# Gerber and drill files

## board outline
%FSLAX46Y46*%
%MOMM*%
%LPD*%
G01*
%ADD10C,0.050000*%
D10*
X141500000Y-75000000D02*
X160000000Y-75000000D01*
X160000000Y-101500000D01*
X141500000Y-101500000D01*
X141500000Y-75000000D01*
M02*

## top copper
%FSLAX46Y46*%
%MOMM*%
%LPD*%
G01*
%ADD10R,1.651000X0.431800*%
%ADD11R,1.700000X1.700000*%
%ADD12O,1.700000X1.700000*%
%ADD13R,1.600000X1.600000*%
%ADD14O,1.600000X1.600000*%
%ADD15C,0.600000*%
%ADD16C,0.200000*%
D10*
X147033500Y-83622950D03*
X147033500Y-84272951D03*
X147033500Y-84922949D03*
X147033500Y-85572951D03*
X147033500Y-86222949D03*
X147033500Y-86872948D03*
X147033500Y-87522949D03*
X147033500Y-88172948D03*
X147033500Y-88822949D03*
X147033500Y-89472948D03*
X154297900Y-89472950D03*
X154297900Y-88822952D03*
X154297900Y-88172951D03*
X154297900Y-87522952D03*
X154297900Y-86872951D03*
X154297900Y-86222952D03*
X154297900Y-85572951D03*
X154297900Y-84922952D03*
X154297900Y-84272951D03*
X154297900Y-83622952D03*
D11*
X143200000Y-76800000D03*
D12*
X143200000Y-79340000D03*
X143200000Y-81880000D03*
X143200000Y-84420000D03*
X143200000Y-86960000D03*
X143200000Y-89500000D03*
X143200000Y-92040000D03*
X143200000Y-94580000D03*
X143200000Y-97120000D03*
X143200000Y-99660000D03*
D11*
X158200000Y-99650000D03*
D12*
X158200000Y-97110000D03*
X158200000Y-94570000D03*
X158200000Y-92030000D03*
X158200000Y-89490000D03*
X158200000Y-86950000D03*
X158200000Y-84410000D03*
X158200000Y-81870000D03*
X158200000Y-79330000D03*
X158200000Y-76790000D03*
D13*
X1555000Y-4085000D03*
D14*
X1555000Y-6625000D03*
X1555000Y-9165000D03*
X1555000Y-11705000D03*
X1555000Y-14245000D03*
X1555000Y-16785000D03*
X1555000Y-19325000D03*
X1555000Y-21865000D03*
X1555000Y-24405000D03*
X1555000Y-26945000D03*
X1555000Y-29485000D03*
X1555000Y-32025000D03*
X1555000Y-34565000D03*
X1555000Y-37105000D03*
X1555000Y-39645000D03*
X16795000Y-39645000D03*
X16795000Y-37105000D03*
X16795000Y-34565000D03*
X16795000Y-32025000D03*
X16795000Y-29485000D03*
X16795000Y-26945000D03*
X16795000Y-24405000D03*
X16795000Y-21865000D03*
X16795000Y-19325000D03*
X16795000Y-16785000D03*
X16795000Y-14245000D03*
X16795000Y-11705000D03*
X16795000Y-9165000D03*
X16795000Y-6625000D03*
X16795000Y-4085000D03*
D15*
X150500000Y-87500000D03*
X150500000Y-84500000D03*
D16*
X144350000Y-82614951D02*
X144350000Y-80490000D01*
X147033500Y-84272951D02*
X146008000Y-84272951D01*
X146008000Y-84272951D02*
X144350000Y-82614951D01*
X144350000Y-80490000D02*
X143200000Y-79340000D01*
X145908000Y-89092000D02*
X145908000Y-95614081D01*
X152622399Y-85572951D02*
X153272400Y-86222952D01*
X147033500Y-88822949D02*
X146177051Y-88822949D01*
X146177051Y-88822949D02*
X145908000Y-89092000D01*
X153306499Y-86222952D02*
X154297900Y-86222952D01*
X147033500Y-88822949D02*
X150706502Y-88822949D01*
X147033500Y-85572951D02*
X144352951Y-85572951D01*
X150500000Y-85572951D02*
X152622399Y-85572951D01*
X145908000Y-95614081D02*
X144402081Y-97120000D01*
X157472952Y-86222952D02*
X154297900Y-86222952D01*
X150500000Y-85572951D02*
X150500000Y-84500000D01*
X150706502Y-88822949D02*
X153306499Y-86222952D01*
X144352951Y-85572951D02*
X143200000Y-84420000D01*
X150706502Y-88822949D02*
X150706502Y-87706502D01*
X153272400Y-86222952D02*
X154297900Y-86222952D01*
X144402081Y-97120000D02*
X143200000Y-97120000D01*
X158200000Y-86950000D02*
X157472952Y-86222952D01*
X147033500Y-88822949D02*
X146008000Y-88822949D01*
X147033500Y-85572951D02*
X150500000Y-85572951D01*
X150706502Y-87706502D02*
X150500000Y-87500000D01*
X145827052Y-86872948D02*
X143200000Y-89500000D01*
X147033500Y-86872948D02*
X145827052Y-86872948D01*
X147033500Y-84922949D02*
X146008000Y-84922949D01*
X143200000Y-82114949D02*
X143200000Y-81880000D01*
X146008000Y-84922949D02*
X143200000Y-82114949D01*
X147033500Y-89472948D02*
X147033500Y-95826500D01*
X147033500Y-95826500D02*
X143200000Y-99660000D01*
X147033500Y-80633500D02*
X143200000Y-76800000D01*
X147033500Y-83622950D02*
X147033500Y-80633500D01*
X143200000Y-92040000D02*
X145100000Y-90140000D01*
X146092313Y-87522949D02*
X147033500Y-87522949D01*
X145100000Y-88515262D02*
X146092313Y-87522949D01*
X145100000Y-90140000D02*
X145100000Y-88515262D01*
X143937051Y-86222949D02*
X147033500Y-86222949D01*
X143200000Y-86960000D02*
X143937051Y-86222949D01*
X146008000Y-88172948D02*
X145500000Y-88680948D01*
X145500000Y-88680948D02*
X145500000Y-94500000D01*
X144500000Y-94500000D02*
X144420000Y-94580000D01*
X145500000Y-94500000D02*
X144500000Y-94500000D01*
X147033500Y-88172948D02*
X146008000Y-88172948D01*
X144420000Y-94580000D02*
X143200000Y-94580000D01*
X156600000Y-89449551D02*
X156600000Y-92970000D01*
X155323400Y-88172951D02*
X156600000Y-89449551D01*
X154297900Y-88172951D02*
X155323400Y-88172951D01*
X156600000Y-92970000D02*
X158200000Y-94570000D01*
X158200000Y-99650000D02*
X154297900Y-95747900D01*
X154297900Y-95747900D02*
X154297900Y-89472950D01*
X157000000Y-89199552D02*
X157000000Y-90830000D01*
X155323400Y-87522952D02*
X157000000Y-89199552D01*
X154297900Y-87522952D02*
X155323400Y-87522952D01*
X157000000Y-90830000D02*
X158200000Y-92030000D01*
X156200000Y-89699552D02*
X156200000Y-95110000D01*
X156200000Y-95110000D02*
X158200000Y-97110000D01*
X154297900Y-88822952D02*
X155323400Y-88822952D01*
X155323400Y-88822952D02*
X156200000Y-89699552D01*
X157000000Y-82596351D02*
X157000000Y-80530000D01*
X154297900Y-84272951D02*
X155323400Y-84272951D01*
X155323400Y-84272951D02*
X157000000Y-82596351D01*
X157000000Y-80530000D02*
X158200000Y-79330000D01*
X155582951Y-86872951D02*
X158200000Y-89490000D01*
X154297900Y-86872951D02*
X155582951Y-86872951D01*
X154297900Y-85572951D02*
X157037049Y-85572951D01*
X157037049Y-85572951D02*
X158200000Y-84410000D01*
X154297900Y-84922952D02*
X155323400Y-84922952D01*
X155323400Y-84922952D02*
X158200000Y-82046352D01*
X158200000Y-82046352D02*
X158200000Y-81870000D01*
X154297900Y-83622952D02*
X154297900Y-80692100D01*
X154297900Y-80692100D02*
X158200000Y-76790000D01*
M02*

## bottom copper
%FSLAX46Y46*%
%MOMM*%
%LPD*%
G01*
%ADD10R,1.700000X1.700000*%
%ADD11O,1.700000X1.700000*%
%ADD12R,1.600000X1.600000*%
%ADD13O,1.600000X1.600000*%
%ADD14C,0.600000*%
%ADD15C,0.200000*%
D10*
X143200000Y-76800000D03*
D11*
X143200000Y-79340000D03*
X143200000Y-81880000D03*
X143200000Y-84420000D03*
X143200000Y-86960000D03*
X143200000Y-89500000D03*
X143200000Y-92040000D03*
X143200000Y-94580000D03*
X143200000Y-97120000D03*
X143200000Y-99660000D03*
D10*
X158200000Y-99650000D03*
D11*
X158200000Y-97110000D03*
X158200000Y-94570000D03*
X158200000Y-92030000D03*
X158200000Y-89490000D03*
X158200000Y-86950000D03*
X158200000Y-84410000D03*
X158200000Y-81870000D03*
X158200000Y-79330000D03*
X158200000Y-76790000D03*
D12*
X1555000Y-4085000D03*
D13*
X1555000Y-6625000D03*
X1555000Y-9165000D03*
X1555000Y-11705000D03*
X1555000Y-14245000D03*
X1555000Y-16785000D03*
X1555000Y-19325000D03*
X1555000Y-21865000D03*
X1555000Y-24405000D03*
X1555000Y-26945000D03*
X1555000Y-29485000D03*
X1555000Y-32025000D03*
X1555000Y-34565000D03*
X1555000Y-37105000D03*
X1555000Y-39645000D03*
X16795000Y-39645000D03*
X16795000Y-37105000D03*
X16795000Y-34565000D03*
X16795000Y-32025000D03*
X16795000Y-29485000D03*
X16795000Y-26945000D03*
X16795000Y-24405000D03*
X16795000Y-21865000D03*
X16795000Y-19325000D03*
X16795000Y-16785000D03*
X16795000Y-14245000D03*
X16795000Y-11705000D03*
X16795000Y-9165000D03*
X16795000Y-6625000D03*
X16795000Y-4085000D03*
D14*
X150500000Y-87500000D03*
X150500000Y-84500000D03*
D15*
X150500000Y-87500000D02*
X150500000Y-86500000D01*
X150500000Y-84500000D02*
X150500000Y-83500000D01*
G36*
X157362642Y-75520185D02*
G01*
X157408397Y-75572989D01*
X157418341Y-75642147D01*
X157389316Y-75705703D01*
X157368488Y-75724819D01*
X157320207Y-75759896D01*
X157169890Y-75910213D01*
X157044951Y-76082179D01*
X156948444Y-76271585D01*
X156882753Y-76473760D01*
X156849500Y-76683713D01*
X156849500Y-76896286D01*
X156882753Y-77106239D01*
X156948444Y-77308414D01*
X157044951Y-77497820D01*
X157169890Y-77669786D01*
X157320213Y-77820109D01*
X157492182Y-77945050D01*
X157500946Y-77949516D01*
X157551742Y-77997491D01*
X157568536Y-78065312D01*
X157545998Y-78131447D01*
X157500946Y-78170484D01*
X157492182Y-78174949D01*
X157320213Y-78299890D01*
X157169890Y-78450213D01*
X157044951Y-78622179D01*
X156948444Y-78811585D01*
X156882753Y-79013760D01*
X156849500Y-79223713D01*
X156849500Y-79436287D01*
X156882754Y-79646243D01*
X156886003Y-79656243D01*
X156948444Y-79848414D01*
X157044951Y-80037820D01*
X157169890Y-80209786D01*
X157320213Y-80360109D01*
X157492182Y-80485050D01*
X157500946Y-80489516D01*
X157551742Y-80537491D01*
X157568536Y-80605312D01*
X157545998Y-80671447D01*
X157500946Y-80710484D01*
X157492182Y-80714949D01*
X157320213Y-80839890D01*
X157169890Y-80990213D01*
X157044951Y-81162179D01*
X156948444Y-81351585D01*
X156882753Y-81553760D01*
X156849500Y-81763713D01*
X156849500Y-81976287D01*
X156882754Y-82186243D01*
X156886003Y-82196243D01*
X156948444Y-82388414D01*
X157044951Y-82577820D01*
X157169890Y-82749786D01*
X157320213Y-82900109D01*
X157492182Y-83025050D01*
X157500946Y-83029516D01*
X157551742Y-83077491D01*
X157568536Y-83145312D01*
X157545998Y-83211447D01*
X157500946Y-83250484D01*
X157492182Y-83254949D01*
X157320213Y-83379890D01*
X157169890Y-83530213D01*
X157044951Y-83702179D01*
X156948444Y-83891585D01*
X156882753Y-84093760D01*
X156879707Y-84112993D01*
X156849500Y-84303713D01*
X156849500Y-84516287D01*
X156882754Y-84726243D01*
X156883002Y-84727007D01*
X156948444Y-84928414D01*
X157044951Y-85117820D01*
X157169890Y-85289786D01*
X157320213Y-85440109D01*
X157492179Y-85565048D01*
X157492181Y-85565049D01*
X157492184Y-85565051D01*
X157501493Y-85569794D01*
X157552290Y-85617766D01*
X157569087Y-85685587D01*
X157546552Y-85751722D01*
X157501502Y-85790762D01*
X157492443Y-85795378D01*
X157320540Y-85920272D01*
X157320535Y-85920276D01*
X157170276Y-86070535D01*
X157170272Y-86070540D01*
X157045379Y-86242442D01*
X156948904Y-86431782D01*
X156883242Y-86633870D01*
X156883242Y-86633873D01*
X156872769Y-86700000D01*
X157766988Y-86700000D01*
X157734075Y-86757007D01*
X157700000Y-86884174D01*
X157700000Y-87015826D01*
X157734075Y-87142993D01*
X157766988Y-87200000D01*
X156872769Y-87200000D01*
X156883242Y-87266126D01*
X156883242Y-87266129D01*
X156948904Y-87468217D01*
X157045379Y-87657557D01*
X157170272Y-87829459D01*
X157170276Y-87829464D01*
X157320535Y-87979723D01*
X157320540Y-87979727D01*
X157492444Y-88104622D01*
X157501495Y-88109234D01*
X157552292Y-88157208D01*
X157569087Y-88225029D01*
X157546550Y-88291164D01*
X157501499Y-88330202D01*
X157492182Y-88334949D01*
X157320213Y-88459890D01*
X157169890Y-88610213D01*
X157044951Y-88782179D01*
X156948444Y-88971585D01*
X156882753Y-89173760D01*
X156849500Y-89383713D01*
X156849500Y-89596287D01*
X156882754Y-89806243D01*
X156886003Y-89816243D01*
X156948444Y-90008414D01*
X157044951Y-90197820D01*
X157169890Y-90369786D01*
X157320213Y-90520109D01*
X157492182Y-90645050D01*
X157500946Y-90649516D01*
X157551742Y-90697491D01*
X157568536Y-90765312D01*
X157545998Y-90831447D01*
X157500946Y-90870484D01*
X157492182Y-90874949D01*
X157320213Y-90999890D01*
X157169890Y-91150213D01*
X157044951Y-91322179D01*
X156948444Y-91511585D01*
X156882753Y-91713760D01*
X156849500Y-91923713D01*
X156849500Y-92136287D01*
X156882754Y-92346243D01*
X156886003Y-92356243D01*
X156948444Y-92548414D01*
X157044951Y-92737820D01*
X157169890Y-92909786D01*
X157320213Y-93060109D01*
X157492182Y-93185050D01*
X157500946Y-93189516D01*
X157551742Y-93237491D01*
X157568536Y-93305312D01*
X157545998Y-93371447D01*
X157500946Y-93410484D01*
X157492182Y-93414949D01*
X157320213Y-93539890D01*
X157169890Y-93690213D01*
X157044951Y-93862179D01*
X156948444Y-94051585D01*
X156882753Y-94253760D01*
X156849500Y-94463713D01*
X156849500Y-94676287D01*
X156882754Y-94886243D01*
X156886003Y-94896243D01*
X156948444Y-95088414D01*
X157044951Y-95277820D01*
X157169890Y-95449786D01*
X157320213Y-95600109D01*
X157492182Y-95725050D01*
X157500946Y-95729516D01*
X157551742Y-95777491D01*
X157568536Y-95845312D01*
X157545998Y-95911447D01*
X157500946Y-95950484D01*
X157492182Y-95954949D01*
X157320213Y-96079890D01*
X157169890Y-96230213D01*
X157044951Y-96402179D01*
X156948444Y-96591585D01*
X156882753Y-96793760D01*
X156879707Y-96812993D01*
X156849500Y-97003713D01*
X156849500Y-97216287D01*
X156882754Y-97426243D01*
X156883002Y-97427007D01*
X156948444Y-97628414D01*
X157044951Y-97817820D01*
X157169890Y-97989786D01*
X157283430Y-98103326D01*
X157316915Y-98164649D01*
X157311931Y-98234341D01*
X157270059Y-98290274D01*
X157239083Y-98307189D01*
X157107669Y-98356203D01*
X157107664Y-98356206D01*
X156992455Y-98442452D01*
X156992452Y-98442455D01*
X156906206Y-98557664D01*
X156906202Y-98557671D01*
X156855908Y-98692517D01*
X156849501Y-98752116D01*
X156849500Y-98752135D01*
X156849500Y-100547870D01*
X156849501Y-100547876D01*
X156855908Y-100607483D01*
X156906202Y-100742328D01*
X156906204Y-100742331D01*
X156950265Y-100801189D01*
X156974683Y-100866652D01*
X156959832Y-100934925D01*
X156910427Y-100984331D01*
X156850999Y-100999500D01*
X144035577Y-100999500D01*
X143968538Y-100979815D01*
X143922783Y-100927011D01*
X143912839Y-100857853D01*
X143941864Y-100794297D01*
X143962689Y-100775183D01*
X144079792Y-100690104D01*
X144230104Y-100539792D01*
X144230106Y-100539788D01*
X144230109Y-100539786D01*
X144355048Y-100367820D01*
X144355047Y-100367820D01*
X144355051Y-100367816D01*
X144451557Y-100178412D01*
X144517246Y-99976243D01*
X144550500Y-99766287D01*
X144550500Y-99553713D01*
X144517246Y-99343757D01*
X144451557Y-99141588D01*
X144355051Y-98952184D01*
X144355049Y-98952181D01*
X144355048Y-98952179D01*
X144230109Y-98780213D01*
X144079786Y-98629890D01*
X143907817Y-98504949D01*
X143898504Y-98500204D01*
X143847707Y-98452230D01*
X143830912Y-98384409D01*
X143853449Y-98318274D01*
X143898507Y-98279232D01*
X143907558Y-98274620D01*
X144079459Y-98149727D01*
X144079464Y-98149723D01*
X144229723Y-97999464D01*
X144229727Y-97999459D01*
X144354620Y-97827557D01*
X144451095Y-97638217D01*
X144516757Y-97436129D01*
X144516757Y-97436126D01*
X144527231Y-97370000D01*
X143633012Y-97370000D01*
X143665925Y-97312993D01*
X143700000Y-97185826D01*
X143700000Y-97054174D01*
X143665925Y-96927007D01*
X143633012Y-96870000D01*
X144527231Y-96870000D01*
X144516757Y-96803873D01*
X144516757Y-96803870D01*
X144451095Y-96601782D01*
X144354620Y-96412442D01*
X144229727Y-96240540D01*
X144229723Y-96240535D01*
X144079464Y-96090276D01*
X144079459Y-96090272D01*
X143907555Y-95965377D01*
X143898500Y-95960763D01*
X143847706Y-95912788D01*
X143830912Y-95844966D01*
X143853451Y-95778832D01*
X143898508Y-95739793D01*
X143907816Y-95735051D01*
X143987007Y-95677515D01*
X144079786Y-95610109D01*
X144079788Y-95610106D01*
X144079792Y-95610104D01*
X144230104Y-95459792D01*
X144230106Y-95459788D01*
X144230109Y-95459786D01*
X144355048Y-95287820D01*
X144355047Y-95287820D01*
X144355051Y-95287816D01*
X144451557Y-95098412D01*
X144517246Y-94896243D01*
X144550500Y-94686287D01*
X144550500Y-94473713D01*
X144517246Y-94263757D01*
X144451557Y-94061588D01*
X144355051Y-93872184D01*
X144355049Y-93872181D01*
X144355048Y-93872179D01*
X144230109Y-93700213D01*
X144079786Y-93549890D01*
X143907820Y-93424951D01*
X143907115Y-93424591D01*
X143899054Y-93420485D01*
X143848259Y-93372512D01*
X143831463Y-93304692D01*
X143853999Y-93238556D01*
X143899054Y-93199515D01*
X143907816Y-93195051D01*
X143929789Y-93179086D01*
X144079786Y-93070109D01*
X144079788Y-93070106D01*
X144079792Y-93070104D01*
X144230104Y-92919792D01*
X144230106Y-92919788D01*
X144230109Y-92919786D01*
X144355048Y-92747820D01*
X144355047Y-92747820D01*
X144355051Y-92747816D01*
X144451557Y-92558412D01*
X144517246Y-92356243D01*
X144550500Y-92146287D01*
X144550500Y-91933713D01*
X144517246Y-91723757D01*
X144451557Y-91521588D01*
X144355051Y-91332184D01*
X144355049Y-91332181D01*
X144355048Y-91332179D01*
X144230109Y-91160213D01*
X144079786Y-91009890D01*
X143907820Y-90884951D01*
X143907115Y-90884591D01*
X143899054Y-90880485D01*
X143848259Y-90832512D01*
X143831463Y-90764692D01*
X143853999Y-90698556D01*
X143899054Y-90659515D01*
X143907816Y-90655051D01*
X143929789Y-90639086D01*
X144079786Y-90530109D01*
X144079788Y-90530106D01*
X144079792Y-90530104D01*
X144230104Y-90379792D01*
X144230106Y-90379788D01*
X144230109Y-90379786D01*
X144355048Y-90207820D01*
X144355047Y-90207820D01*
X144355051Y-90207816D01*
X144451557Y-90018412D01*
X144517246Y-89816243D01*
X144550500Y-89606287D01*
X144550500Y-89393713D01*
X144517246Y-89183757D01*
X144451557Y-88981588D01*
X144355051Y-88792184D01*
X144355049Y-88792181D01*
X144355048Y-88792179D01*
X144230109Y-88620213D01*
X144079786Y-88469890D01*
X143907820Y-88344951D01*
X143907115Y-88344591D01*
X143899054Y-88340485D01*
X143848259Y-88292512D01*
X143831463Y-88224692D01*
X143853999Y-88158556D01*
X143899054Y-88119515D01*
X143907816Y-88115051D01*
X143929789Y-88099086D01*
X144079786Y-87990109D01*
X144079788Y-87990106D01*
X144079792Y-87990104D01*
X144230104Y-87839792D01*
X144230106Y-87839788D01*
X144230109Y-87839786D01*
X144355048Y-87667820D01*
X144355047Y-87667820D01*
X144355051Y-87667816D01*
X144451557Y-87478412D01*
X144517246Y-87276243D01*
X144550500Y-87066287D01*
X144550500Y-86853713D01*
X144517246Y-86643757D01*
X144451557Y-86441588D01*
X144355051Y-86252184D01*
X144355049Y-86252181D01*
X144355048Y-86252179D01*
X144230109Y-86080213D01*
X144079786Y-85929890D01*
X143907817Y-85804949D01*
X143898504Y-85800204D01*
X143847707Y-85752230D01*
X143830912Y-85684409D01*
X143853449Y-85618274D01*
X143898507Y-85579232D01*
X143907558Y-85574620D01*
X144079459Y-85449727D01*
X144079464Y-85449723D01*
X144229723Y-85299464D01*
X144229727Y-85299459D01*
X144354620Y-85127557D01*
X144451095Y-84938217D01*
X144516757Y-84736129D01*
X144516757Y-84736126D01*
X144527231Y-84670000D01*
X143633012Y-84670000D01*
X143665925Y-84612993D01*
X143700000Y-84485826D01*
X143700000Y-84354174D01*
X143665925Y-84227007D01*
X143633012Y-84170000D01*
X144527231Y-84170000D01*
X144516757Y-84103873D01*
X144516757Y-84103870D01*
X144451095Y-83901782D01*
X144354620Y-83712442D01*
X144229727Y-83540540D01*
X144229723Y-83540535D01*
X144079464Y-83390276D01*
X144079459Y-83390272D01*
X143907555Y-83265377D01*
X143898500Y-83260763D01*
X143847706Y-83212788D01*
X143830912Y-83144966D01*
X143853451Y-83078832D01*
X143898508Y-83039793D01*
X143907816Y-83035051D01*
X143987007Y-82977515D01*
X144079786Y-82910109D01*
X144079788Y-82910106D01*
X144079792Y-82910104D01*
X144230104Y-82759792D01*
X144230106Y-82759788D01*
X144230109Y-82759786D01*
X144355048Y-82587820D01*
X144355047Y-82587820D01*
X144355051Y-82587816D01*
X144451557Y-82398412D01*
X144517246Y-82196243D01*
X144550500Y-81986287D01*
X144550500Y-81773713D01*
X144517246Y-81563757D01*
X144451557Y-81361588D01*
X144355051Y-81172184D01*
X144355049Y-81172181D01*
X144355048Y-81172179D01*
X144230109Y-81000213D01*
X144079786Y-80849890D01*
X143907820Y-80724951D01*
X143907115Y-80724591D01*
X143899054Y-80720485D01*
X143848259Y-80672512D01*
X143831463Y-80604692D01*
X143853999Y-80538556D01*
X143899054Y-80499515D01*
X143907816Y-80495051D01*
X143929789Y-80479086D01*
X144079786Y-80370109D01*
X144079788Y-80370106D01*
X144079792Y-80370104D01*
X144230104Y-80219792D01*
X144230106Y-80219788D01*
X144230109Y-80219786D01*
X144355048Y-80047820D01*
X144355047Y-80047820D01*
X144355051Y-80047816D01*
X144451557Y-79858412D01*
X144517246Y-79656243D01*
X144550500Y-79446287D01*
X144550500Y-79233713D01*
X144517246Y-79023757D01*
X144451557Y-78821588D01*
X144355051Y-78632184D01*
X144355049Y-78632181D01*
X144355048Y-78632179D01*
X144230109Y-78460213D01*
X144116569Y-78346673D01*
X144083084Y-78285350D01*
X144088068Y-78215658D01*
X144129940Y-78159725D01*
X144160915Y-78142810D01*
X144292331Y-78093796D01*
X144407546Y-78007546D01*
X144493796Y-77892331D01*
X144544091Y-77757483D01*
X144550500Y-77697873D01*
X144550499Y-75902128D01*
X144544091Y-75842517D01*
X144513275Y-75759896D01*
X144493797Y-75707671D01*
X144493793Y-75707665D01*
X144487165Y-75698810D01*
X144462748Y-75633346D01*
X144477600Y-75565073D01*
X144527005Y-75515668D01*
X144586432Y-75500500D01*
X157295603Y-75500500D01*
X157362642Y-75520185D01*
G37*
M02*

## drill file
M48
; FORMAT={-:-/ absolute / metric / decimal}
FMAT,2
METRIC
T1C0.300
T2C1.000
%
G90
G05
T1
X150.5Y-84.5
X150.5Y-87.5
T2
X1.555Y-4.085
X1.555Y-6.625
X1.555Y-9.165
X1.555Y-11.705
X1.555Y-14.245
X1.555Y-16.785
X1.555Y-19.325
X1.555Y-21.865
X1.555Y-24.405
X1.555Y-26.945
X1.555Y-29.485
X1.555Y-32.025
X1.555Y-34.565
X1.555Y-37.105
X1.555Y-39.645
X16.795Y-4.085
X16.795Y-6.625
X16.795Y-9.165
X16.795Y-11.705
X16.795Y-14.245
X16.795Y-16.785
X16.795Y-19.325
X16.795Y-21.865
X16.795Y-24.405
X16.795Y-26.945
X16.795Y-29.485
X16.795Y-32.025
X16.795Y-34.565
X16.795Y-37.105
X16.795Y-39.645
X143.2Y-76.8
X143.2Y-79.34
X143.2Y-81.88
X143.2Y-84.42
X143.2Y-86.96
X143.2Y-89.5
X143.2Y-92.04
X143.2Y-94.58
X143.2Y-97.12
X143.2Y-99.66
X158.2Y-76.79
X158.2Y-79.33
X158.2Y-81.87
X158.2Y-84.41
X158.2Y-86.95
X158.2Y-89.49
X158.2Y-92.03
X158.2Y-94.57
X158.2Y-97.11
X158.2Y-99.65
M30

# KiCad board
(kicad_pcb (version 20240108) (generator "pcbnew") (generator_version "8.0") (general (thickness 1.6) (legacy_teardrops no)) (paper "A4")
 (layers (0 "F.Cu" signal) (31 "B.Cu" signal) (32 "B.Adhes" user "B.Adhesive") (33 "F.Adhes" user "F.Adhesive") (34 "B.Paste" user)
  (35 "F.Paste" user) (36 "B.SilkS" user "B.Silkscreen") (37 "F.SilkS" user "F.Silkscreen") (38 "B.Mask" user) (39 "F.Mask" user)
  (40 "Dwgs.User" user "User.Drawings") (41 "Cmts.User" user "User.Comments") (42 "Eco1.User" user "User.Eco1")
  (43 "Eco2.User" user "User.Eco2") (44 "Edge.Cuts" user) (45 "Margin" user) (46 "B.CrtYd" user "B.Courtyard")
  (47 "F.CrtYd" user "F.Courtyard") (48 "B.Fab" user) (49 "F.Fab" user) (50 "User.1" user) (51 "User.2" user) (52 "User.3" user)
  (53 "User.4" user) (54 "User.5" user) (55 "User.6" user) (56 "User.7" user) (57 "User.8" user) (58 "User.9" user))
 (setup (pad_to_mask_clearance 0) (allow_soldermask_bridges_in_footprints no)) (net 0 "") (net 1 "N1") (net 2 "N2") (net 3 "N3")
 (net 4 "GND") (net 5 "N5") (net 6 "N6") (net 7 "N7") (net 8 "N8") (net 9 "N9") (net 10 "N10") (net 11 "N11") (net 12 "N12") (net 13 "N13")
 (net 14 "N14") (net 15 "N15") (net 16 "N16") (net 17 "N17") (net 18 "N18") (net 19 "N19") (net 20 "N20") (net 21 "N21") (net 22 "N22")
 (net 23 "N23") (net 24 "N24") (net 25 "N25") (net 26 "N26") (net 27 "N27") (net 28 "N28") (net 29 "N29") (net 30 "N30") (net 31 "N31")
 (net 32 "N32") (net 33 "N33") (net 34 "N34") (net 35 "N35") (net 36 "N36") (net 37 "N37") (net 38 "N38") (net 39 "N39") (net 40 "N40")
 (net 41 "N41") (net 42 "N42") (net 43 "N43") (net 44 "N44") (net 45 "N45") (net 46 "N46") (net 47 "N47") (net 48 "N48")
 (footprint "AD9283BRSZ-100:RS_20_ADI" (layer "F.Cu") (at 150.6657 86.54795)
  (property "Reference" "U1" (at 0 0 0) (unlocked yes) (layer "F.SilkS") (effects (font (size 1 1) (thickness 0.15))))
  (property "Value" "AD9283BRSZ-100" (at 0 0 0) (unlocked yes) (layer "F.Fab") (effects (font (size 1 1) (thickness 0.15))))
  (pad "1" smd rect (at -3.6322 -2.925) (size 1.651 0.4318) (layers "F.Cu" "F.Paste" "F.Mask") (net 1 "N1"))
  (pad "2" smd rect (at -3.6322 -2.274999) (size 1.651 0.4318) (layers "F.Cu" "F.Paste" "F.Mask") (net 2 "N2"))
  (pad "3" smd rect (at -3.6322 -1.625001) (size 1.651 0.4318) (layers "F.Cu" "F.Paste" "F.Mask") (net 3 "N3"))
  (pad "4" smd rect (at -3.6322 -0.974999) (size 1.651 0.4318) (layers "F.Cu" "F.Paste" "F.Mask") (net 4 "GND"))
  (pad "5" smd rect (at -3.6322 -0.325001) (size 1.651 0.4318) (layers "F.Cu" "F.Paste" "F.Mask") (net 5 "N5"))
  (pad "6" smd rect (at -3.6322 0.324998) (size 1.651 0.4318) (layers "F.Cu" "F.Paste" "F.Mask") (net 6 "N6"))
  (pad "7" smd rect (at -3.6322 0.974999) (size 1.651 0.4318) (layers "F.Cu" "F.Paste" "F.Mask") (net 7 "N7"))
  (pad "8" smd rect (at -3.6322 1.624998) (size 1.651 0.4318) (layers "F.Cu" "F.Paste" "F.Mask") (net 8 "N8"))
  (pad "9" smd rect (at -3.6322 2.274999) (size 1.651 0.4318) (layers "F.Cu" "F.Paste" "F.Mask") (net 4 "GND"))
  (pad "10" smd rect (at -3.6322 2.924998) (size 1.651 0.4318) (layers "F.Cu" "F.Paste" "F.Mask") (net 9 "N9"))
  (pad "11" smd rect (at 3.6322 2.925) (size 1.651 0.4318) (layers "F.Cu" "F.Paste" "F.Mask") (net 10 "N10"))
  (pad "12" smd rect (at 3.6322 2.275002) (size 1.651 0.4318) (layers "F.Cu" "F.Paste" "F.Mask") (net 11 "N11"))
  (pad "13" smd rect (at 3.6322 1.625001) (size 1.651 0.4318) (layers "F.Cu" "F.Paste" "F.Mask") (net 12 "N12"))
  (pad "14" smd rect (at 3.6322 0.975002) (size 1.651 0.4318) (layers "F.Cu" "F.Paste" "F.Mask") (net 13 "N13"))
  (pad "15" smd rect (at 3.6322 0.325001) (size 1.651 0.4318) (layers "F.Cu" "F.Paste" "F.Mask") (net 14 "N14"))
  (pad "16" smd rect (at 3.6322 -0.324998) (size 1.651 0.4318) (layers "F.Cu" "F.Paste" "F.Mask") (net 4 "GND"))
  (pad "17" smd rect (at 3.6322 -0.974999) (size 1.651 0.4318) (layers "F.Cu" "F.Paste" "F.Mask") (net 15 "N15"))
  (pad "18" smd rect (at 3.6322 -1.624998) (size 1.651 0.4318) (layers "F.Cu" "F.Paste" "F.Mask") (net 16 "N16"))
  (pad "19" smd rect (at 3.6322 -2.274999) (size 1.651 0.4318) (layers "F.Cu" "F.Paste" "F.Mask") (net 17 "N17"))
  (pad "20" smd rect (at 3.6322 -2.924998) (size 1.651 0.4318) (layers "F.Cu" "F.Paste" "F.Mask") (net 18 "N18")))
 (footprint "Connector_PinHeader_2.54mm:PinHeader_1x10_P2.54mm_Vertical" (layer "F.Cu") (at 143.2 76.8)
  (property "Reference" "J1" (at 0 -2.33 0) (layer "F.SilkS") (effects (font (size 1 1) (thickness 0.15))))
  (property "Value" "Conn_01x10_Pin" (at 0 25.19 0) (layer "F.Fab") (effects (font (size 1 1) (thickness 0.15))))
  (pad "1" thru_hole rect (at 0 0) (size 1.7 1.7) (drill 1) (layers "*.Cu" "*.Mask") (remove_unused_layers no) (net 1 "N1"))
  (pad "2" thru_hole oval (at 0 2.54) (size 1.7 1.7) (drill 1) (layers "*.Cu" "*.Mask") (remove_unused_layers no) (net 2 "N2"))
  (pad "3" thru_hole oval (at 0 5.08) (size 1.7 1.7) (drill 1) (layers "*.Cu" "*.Mask") (remove_unused_layers no) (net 3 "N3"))
  (pad "4" thru_hole oval (at 0 7.62) (size 1.7 1.7) (drill 1) (layers "*.Cu" "*.Mask") (remove_unused_layers no) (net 4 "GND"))
  (pad "5" thru_hole oval (at 0 10.16) (size 1.7 1.7) (drill 1) (layers "*.Cu" "*.Mask") (remove_unused_layers no) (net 5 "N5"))
  (pad "6" thru_hole oval (at 0 12.7) (size 1.7 1.7) (drill 1) (layers "*.Cu" "*.Mask") (remove_unused_layers no) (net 6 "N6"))
  (pad "7" thru_hole oval (at 0 15.24) (size 1.7 1.7) (drill 1) (layers "*.Cu" "*.Mask") (remove_unused_layers no) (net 7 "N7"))
  (pad "8" thru_hole oval (at 0 17.78) (size 1.7 1.7) (drill 1) (layers "*.Cu" "*.Mask") (remove_unused_layers no) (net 8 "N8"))
  (pad "9" thru_hole oval (at 0 20.32) (size 1.7 1.7) (drill 1) (layers "*.Cu" "*.Mask") (remove_unused_layers no) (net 4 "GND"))
  (pad "10" thru_hole oval (at 0 22.86) (size 1.7 1.7) (drill 1) (layers "*.Cu" "*.Mask") (remove_unused_layers no) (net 9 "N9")))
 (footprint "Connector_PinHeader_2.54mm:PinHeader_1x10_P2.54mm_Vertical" (layer "F.Cu") (at 158.2 99.65 180)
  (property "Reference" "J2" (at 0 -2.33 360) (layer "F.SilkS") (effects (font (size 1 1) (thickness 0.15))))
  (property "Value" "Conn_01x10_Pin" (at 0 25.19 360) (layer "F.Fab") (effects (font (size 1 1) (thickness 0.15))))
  (pad "1" thru_hole rect (at 0 0 180) (size 1.7 1.7) (drill 1) (layers "*.Cu" "*.Mask") (remove_unused_layers no) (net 10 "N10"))
  (pad "2" thru_hole oval (at 0 2.54 180) (size 1.7 1.7) (drill 1) (layers "*.Cu" "*.Mask") (remove_unused_layers no) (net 11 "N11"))
  (pad "3" thru_hole oval (at 0 5.08 180) (size 1.7 1.7) (drill 1) (layers "*.Cu" "*.Mask") (remove_unused_layers no) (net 12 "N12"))
  (pad "4" thru_hole oval (at 0 7.62 180) (size 1.7 1.7) (drill 1) (layers "*.Cu" "*.Mask") (remove_unused_layers no) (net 13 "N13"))
  (pad "5" thru_hole oval (at 0 10.16 180) (size 1.7 1.7) (drill 1) (layers "*.Cu" "*.Mask") (remove_unused_layers no) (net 14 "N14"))
  (pad "6" thru_hole oval (at 0 12.7 180) (size 1.7 1.7) (drill 1) (layers "*.Cu" "*.Mask") (remove_unused_layers no) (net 4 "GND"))
  (pad "7" thru_hole oval (at 0 15.24 180) (size 1.7 1.7) (drill 1) (layers "*.Cu" "*.Mask") (remove_unused_layers no) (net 15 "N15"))
  (pad "8" thru_hole oval (at 0 17.78 180) (size 1.7 1.7) (drill 1) (layers "*.Cu" "*.Mask") (remove_unused_layers no) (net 16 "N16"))
  (pad "9" thru_hole oval (at 0 20.32 180) (size 1.7 1.7) (drill 1) (layers "*.Cu" "*.Mask") (remove_unused_layers no) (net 17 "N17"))
  (pad "10" thru_hole oval (at 0 22.86 180) (size 1.7 1.7) (drill 1) (layers "*.Cu" "*.Mask") (remove_unused_layers no) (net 18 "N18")))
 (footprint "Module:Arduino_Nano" (layer "F.Cu") (at 1.555 4.085)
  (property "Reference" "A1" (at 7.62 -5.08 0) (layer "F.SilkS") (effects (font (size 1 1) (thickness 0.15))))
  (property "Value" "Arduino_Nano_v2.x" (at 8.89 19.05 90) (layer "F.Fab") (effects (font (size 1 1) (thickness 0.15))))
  (pad "1" thru_hole rect (at 0 0) (size 1.6 1.6) (drill 1) (layers "*.Cu" "*.Mask") (remove_unused_layers no) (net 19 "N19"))
  (pad "2" thru_hole oval (at 0 2.54) (size 1.6 1.6) (drill 1) (layers "*.Cu" "*.Mask") (remove_unused_layers no) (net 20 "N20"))
  (pad "3" thru_hole oval (at 0 5.08) (size 1.6 1.6) (drill 1) (layers "*.Cu" "*.Mask") (remove_unused_layers no) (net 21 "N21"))
  (pad "4" thru_hole oval (at 0 7.62) (size 1.6 1.6) (drill 1) (layers "*.Cu" "*.Mask") (remove_unused_layers no) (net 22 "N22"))
  (pad "5" thru_hole oval (at 0 10.16) (size 1.6 1.6) (drill 1) (layers "*.Cu" "*.Mask") (remove_unused_layers no) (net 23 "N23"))
  (pad "6" thru_hole oval (at 0 12.7) (size 1.6 1.6) (drill 1) (layers "*.Cu" "*.Mask") (remove_unused_layers no) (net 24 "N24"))
  (pad "7" thru_hole oval (at 0 15.24) (size 1.6 1.6) (drill 1) (layers "*.Cu" "*.Mask") (remove_unused_layers no) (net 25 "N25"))
  (pad "8" thru_hole oval (at 0 17.78) (size 1.6 1.6) (drill 1) (layers "*.Cu" "*.Mask") (remove_unused_layers no) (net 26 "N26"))
  (pad "9" thru_hole oval (at 0 20.32) (size 1.6 1.6) (drill 1) (layers "*.Cu" "*.Mask") (remove_unused_layers no) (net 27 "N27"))
  (pad "10" thru_hole oval (at 0 22.86) (size 1.6 1.6) (drill 1) (layers "*.Cu" "*.Mask") (remove_unused_layers no) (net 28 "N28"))
  (pad "11" thru_hole oval (at 0 25.4) (size 1.6 1.6) (drill 1) (layers "*.Cu" "*.Mask") (remove_unused_layers no) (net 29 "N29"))
  (pad "12" thru_hole oval (at 0 27.94) (size 1.6 1.6) (drill 1) (layers "*.Cu" "*.Mask") (remove_unused_layers no) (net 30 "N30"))
  (pad "13" thru_hole oval (at 0 30.48) (size 1.6 1.6) (drill 1) (layers "*.Cu" "*.Mask") (remove_unused_layers no) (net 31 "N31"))
  (pad "14" thru_hole oval (at 0 33.02) (size 1.6 1.6) (drill 1) (layers "*.Cu" "*.Mask") (remove_unused_layers no) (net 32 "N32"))
  (pad "15" thru_hole oval (at 0 35.56) (size 1.6 1.6) (drill 1) (layers "*.Cu" "*.Mask") (remove_unused_layers no) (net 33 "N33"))
  (pad "16" thru_hole oval (at 15.24 35.56) (size 1.6 1.6) (drill 1) (layers "*.Cu" "*.Mask") (remove_unused_layers no) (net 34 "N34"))
  (pad "17" thru_hole oval (at 15.24 33.02) (size 1.6 1.6) (drill 1) (layers "*.Cu" "*.Mask") (remove_unused_layers no) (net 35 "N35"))
  (pad "18" thru_hole oval (at 15.24 30.48) (size 1.6 1.6) (drill 1) (layers "*.Cu" "*.Mask") (remove_unused_layers no) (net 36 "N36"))
  (pad "19" thru_hole oval (at 15.24 27.94) (size 1.6 1.6) (drill 1) (layers "*.Cu" "*.Mask") (remove_unused_layers no) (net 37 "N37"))
  (pad "20" thru_hole oval (at 15.24 25.4) (size 1.6 1.6) (drill 1) (layers "*.Cu" "*.Mask") (remove_unused_layers no) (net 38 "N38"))
  (pad "21" thru_hole oval (at 15.24 22.86) (size 1.6 1.6) (drill 1) (layers "*.Cu" "*.Mask") (remove_unused_layers no) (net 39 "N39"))
  (pad "22" thru_hole oval (at 15.24 20.32) (size 1.6 1.6) (drill 1) (layers "*.Cu" "*.Mask") (remove_unused_layers no) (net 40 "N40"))
  (pad "23" thru_hole oval (at 15.24 17.78) (size 1.6 1.6) (drill 1) (layers "*.Cu" "*.Mask") (remove_unused_layers no) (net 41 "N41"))
  (pad "24" thru_hole oval (at 15.24 15.24) (size 1.6 1.6) (drill 1) (layers "*.Cu" "*.Mask") (remove_unused_layers no) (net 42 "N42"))
  (pad "25" thru_hole oval (at 15.24 12.7) (size 1.6 1.6) (drill 1) (layers "*.Cu" "*.Mask") (remove_unused_layers no) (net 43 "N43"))
  (pad "26" thru_hole oval (at 15.24 10.16) (size 1.6 1.6) (drill 1) (layers "*.Cu" "*.Mask") (remove_unused_layers no) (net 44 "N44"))
  (pad "27" thru_hole oval (at 15.24 7.62) (size 1.6 1.6) (drill 1) (layers "*.Cu" "*.Mask") (remove_unused_layers no) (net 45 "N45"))
  (pad "28" thru_hole oval (at 15.24 5.08) (size 1.6 1.6) (drill 1) (layers "*.Cu" "*.Mask") (remove_unused_layers no) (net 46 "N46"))
  (pad "29" thru_hole oval (at 15.24 2.54) (size 1.6 1.6) (drill 1) (layers "*.Cu" "*.Mask") (remove_unused_layers no) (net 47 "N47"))
  (pad "30" thru_hole oval (at 15.24 0) (size 1.6 1.6) (drill 1) (layers "*.Cu" "*.Mask") (remove_unused_layers no) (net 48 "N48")))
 (gr_rect (start 141.5 75) (end 160 101.5) (stroke (width 0.05) (type default)) (fill none) (layer "Edge.Cuts"))
 (segment (start 144.35 82.614951) (end 144.35 80.49) (width 0.2) (layer "F.Cu") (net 2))
 (segment (start 147.0335 84.272951) (end 146.008 84.272951) (width 0.2) (layer "F.Cu") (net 2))
 (segment (start 146.008 84.272951) (end 144.35 82.614951) (width 0.2) (layer "F.Cu") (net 2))
 (segment (start 144.35 80.49) (end 143.2 79.34) (width 0.2) (layer "F.Cu") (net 2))
 (segment (start 145.908 89.092) (end 145.908 95.614081) (width 0.2) (layer "F.Cu") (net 4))
 (segment (start 152.622399 85.572951) (end 153.2724 86.222952) (width 0.2) (layer "F.Cu") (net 4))
 (segment (start 147.0335 88.822949) (end 146.177051 88.822949) (width 0.2) (layer "F.Cu") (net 4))
 (segment (start 146.177051 88.822949) (end 145.908 89.092) (width 0.2) (layer "F.Cu") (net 4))
 (segment (start 153.306499 86.222952) (end 154.2979 86.222952) (width 0.2) (layer "F.Cu") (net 4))
 (segment (start 147.0335 88.822949) (end 150.706502 88.822949) (width 0.2) (layer "F.Cu") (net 4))
 (segment (start 147.0335 85.572951) (end 144.352951 85.572951) (width 0.2) (layer "F.Cu") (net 4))
 (segment (start 150.5 85.572951) (end 152.622399 85.572951) (width 0.2) (layer "F.Cu") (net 4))
 (segment (start 145.908 95.614081) (end 144.402081 97.12) (width 0.2) (layer "F.Cu") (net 4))
 (segment (start 157.472952 86.222952) (end 154.2979 86.222952) (width 0.2) (layer "F.Cu") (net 4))
 (segment (start 150.5 85.572951) (end 150.5 84.5) (width 0.2) (layer "F.Cu") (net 4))
 (segment (start 150.706502 88.822949) (end 153.306499 86.222952) (width 0.2) (layer "F.Cu") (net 4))
 (segment (start 144.352951 85.572951) (end 143.2 84.42) (width 0.2) (layer "F.Cu") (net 4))
 (segment (start 150.706502 88.822949) (end 150.706502 87.706502) (width 0.2) (layer "F.Cu") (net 4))
 (segment (start 153.2724 86.222952) (end 154.2979 86.222952) (width 0.2) (layer "F.Cu") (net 4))
 (segment (start 144.402081 97.12) (end 143.2 97.12) (width 0.2) (layer "F.Cu") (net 4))
 (segment (start 158.2 86.95) (end 157.472952 86.222952) (width 0.2) (layer "F.Cu") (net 4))
 (segment (start 147.0335 88.822949) (end 146.008 88.822949) (width 0.2) (layer "F.Cu") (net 4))
 (segment (start 147.0335 85.572951) (end 150.5 85.572951) (width 0.2) (layer "F.Cu") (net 4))
 (segment (start 150.706502 87.706502) (end 150.5 87.5) (width 0.2) (layer "F.Cu") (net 4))
 (via (at 150.5 87.5) (size 0.6) (drill 0.3) (layers "F.Cu" "B.Cu") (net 4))
 (via (at 150.5 84.5) (size 0.6) (drill 0.3) (layers "F.Cu" "B.Cu") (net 4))
 (segment (start 150.5 87.5) (end 150.5 86.5) (width 0.2) (layer "B.Cu") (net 4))
 (segment (start 150.5 84.5) (end 150.5 83.5) (width 0.2) (layer "B.Cu") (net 4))
 (segment (start 145.827052 86.872948) (end 143.2 89.5) (width 0.2) (layer "F.Cu") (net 6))
 (segment (start 147.0335 86.872948) (end 145.827052 86.872948) (width 0.2) (layer "F.Cu") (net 6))
 (segment (start 147.0335 84.922949) (end 146.008 84.922949) (width 0.2) (layer "F.Cu") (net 3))
 (segment (start 143.2 82.114949) (end 143.2 81.88) (width 0.2) (layer "F.Cu") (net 3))
 (segment (start 146.008 84.922949) (end 143.2 82.114949) (width 0.2) (layer "F.Cu") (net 3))
 (segment (start 147.0335 89.472948) (end 147.0335 95.8265) (width 0.2) (layer "F.Cu") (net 9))
 (segment (start 147.0335 95.8265) (end 143.2 99.66) (width 0.2) (layer "F.Cu") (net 9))
 (segment (start 147.0335 80.6335) (end 143.2 76.8) (width 0.2) (layer "F.Cu") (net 1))
 (segment (start 147.0335 83.62295) (end 147.0335 80.6335) (width 0.2) (layer "F.Cu") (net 1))
 (segment (start 143.2 92.04) (end 145.1 90.14) (width 0.2) (layer "F.Cu") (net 7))
 (segment (start 146.092313 87.522949) (end 147.0335 87.522949) (width 0.2) (layer "F.Cu") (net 7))
 (segment (start 145.1 88.515262) (end 146.092313 87.522949) (width 0.2) (layer "F.Cu") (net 7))
 (segment (start 145.1 90.14) (end 145.1 88.515262) (width 0.2) (layer "F.Cu") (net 7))
 (segment (start 143.937051 86.222949) (end 147.0335 86.222949) (width 0.2) (layer "F.Cu") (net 5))
 (segment (start 143.2 86.96) (end 143.937051 86.222949) (width 0.2) (layer "F.Cu") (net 5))
 (segment (start 146.008 88.172948) (end 145.5 88.680948) (width 0.2) (layer "F.Cu") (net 8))
 (segment (start 145.5 88.680948) (end 145.5 94.5) (width 0.2) (layer "F.Cu") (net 8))
 (segment (start 144.5 94.5) (end 144.42 94.58) (width 0.2) (layer "F.Cu") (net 8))
 (segment (start 145.5 94.5) (end 144.5 94.5) (width 0.2) (layer "F.Cu") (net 8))
 (segment (start 147.0335 88.172948) (end 146.008 88.172948) (width 0.2) (layer "F.Cu") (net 8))
 (segment (start 144.42 94.58) (end 143.2 94.58) (width 0.2) (layer "F.Cu") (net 8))
 (segment (start 156.6 89.449551) (end 156.6 92.97) (width 0.2) (layer "F.Cu") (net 12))
 (segment (start 155.3234 88.172951) (end 156.6 89.449551) (width 0.2) (layer "F.Cu") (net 12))
 (segment (start 154.2979 88.172951) (end 155.3234 88.172951) (width 0.2) (layer "F.Cu") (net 12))
 (segment (start 156.6 92.97) (end 158.2 94.57) (width 0.2) (layer "F.Cu") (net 12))
 (segment (start 158.2 99.65) (end 154.2979 95.7479) (width 0.2) (layer "F.Cu") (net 10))
 (segment (start 154.2979 95.7479) (end 154.2979 89.47295) (width 0.2) (layer "F.Cu") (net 10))
 (segment (start 157 89.199552) (end 157 90.83) (width 0.2) (layer "F.Cu") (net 13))
 (segment (start 155.3234 87.522952) (end 157 89.199552) (width 0.2) (layer "F.Cu") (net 13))
 (segment (start 154.2979 87.522952) (end 155.3234 87.522952) (width 0.2) (layer "F.Cu") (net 13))
 (segment (start 157 90.83) (end 158.2 92.03) (width 0.2) (layer "F.Cu") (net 13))
 (segment (start 156.2 89.699552) (end 156.2 95.11) (width 0.2) (layer "F.Cu") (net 11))
 (segment (start 156.2 95.11) (end 158.2 97.11) (width 0.2) (layer "F.Cu") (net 11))
 (segment (start 154.2979 88.822952) (end 155.3234 88.822952) (width 0.2) (layer "F.Cu") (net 11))
 (segment (start 155.3234 88.822952) (end 156.2 89.699552) (width 0.2) (layer "F.Cu") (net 11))
 (segment (start 157 82.596351) (end 157 80.53) (width 0.2) (layer "F.Cu") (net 17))
 (segment (start 154.2979 84.272951) (end 155.3234 84.272951) (width 0.2) (layer "F.Cu") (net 17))
 (segment (start 155.3234 84.272951) (end 157 82.596351) (width 0.2) (layer "F.Cu") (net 17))
 (segment (start 157 80.53) (end 158.2 79.33) (width 0.2) (layer "F.Cu") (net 17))
 (segment (start 155.582951 86.872951) (end 158.2 89.49) (width 0.2) (layer "F.Cu") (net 14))
 (segment (start 154.2979 86.872951) (end 155.582951 86.872951) (width 0.2) (layer "F.Cu") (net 14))
 (segment (start 154.2979 85.572951) (end 157.037049 85.572951) (width 0.2) (layer "F.Cu") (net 15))
 (segment (start 157.037049 85.572951) (end 158.2 84.41) (width 0.2) (layer "F.Cu") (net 15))
 (segment (start 154.2979 84.922952) (end 155.3234 84.922952) (width 0.2) (layer "F.Cu") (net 16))
 (segment (start 155.3234 84.922952) (end 158.2 82.046352) (width 0.2) (layer "F.Cu") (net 16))
 (segment (start 158.2 82.046352) (end 158.2 81.87) (width 0.2) (layer "F.Cu") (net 16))
 (segment (start 154.2979 83.622952) (end 154.2979 80.6921) (width 0.2) (layer "F.Cu") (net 18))
 (segment (start 154.2979 80.6921) (end 158.2 76.79) (width 0.2) (layer "F.Cu") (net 18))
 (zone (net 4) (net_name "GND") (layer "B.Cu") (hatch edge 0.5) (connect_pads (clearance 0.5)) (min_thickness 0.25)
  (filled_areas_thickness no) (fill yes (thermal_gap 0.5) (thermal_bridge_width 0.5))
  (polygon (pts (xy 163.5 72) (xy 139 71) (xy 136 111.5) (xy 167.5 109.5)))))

